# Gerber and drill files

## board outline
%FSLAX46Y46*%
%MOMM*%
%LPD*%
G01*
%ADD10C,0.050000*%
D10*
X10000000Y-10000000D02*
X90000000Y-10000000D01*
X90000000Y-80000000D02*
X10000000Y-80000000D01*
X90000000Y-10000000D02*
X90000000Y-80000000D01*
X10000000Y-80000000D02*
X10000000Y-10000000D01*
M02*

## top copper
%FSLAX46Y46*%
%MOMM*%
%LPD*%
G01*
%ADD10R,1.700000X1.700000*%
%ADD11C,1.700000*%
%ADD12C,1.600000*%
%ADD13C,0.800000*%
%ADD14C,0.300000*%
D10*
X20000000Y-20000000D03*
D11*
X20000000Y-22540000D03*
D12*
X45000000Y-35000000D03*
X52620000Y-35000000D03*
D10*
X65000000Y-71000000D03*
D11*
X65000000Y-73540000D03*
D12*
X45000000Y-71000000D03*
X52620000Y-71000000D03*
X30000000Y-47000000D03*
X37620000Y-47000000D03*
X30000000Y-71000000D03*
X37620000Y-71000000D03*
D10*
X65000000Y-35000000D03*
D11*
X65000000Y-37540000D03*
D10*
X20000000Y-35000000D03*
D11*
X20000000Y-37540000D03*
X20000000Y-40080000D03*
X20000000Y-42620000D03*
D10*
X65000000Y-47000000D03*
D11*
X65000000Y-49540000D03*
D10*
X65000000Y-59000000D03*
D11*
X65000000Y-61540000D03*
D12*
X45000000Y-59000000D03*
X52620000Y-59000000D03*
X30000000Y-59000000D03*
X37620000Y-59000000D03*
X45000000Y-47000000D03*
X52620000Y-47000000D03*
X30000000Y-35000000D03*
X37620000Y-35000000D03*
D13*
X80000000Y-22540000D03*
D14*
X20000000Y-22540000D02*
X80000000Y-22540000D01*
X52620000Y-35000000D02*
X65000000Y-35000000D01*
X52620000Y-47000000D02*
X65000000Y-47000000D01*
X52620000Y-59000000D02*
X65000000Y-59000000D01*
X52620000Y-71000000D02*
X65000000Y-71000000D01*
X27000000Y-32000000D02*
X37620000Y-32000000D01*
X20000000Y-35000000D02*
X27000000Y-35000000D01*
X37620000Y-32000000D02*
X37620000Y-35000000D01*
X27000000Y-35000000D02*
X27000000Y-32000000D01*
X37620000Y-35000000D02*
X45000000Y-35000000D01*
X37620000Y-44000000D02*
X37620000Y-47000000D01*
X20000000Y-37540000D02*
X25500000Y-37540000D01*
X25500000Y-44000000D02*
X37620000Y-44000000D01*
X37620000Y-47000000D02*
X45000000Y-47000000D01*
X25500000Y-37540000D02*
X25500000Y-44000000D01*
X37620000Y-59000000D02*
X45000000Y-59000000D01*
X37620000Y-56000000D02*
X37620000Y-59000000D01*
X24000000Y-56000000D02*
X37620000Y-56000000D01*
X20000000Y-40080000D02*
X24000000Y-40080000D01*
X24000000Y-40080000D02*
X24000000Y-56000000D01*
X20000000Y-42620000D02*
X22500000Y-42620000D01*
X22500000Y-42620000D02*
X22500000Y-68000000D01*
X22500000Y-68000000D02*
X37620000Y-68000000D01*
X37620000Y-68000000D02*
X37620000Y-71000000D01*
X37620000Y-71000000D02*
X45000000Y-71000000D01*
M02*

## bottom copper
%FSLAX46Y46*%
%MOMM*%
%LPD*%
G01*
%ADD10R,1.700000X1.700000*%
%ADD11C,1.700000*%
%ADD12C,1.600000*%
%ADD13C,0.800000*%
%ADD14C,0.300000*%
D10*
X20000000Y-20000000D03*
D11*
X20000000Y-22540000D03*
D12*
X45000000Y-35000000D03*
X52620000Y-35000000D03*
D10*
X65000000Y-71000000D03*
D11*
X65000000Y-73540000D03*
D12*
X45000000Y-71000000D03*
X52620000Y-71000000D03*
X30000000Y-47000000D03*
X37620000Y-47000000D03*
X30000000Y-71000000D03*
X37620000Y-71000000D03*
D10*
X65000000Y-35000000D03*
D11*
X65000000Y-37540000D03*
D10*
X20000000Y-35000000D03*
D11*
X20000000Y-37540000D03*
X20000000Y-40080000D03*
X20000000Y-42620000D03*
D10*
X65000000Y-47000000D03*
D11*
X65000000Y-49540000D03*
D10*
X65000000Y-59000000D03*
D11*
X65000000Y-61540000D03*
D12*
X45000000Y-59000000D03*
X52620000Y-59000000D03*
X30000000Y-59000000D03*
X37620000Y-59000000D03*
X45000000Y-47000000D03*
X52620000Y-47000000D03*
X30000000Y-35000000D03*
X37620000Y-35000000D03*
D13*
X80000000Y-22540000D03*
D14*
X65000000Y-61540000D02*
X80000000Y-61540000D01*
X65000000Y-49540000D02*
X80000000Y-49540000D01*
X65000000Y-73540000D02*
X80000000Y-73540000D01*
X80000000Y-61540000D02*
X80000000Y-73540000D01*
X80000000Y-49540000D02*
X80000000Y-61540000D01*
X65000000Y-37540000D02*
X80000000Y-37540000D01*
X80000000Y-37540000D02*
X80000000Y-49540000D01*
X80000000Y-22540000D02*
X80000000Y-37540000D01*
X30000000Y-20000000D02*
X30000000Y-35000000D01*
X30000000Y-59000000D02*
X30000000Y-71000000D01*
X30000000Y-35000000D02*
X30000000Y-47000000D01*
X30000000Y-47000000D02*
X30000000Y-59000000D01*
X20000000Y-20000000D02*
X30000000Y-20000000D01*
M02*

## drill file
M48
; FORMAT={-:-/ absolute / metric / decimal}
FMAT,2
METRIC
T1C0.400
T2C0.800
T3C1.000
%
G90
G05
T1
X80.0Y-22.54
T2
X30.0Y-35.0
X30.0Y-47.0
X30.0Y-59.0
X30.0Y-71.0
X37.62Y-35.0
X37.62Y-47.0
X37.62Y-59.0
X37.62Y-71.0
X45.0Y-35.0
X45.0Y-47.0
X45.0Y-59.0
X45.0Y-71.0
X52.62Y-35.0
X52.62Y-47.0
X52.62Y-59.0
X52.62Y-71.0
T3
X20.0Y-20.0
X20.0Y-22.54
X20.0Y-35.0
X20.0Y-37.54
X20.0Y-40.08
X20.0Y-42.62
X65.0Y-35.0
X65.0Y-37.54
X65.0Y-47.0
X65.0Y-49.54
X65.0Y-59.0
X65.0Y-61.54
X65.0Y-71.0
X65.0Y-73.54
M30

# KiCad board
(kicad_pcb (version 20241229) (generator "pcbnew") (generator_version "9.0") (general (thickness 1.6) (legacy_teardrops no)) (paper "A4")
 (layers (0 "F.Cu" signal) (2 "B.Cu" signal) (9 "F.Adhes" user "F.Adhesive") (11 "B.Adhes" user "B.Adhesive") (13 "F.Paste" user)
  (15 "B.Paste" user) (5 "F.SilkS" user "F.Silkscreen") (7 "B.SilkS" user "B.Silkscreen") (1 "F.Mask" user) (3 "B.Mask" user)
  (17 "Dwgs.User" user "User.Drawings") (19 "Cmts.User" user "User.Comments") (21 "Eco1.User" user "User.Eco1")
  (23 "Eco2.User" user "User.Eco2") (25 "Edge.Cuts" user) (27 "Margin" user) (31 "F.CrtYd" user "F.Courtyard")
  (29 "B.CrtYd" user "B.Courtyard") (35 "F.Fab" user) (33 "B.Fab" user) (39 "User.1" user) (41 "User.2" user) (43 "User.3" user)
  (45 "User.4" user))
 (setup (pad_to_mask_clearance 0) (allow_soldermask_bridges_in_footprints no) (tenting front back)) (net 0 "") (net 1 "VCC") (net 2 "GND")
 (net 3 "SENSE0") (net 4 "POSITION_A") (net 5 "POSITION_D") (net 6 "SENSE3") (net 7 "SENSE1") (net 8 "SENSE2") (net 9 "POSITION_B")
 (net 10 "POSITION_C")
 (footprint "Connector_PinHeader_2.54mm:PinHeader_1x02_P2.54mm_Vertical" (layer "F.Cu") (at 20 20)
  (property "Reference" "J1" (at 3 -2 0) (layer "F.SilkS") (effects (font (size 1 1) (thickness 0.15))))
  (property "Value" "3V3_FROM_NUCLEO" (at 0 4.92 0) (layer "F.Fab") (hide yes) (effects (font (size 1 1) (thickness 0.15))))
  (pad "1" thru_hole rect (at 0 0) (size 1.7 1.7) (drill 1) (layers "*.Cu" "*.Mask") (remove_unused_layers no) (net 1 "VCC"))
  (pad "2" thru_hole circle (at 0 2.54) (size 1.7 1.7) (drill 1) (layers "*.Cu" "*.Mask") (remove_unused_layers no) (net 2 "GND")))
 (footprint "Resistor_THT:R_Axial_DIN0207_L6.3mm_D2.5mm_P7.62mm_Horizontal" (layer "F.Cu") (at 45 35)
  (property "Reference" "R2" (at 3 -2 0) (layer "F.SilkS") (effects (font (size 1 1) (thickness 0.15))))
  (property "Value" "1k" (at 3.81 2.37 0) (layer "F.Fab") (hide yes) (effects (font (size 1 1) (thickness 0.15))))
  (pad "1" thru_hole circle (at 0 0) (size 1.6 1.6) (drill 0.8) (layers "*.Cu" "*.Mask") (remove_unused_layers no) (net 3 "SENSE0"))
  (pad "2" thru_hole circle (at 7.62 0) (size 1.6 1.6) (drill 0.8) (layers "*.Cu" "*.Mask") (remove_unused_layers no) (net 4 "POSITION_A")))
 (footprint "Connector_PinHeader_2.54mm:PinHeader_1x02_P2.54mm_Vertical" (layer "F.Cu") (at 65 71)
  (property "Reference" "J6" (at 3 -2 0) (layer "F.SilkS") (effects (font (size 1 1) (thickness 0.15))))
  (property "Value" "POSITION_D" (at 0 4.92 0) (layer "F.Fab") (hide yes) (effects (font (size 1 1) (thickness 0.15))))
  (pad "1" thru_hole rect (at 0 0) (size 1.7 1.7) (drill 1) (layers "*.Cu" "*.Mask") (remove_unused_layers no) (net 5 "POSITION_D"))
  (pad "2" thru_hole circle (at 0 2.54) (size 1.7 1.7) (drill 1) (layers "*.Cu" "*.Mask") (remove_unused_layers no) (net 2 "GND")))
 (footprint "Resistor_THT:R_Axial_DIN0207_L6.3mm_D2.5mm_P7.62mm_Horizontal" (layer "F.Cu") (at 45 71)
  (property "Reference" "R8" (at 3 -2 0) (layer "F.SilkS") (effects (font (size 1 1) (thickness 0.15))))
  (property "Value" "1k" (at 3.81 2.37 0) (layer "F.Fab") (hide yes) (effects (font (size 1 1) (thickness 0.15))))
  (pad "1" thru_hole circle (at 0 0) (size 1.6 1.6) (drill 0.8) (layers "*.Cu" "*.Mask") (remove_unused_layers no) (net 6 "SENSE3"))
  (pad "2" thru_hole circle (at 7.62 0) (size 1.6 1.6) (drill 0.8) (layers "*.Cu" "*.Mask") (remove_unused_layers no) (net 5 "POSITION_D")))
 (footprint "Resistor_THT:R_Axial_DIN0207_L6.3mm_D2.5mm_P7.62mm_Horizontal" (layer "F.Cu") (at 30 47)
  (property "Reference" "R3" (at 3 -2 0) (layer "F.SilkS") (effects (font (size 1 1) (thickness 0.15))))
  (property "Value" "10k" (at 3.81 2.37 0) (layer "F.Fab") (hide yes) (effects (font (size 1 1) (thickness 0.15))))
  (pad "1" thru_hole circle (at 0 0) (size 1.6 1.6) (drill 0.8) (layers "*.Cu" "*.Mask") (remove_unused_layers no) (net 1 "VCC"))
  (pad "2" thru_hole circle (at 7.62 0) (size 1.6 1.6) (drill 0.8) (layers "*.Cu" "*.Mask") (remove_unused_layers no) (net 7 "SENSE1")))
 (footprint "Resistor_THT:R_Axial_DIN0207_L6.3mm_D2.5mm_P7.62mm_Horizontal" (layer "F.Cu") (at 30 71)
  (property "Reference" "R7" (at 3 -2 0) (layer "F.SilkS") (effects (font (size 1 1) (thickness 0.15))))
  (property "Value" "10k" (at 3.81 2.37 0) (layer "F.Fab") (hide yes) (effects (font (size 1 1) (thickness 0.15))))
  (pad "1" thru_hole circle (at 0 0) (size 1.6 1.6) (drill 0.8) (layers "*.Cu" "*.Mask") (remove_unused_layers no) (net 1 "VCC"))
  (pad "2" thru_hole circle (at 7.62 0) (size 1.6 1.6) (drill 0.8) (layers "*.Cu" "*.Mask") (remove_unused_layers no) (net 6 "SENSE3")))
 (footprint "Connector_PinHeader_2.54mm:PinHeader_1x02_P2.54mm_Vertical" (layer "F.Cu") (at 65 35)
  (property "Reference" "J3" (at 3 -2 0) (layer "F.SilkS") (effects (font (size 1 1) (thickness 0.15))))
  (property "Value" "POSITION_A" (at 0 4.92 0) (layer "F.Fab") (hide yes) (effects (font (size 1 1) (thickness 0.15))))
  (pad "1" thru_hole rect (at 0 0) (size 1.7 1.7) (drill 1) (layers "*.Cu" "*.Mask") (remove_unused_layers no) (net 4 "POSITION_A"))
  (pad "2" thru_hole circle (at 0 2.54) (size 1.7 1.7) (drill 1) (layers "*.Cu" "*.Mask") (remove_unused_layers no) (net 2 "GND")))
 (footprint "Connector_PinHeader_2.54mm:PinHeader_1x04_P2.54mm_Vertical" (layer "F.Cu") (at 20 35)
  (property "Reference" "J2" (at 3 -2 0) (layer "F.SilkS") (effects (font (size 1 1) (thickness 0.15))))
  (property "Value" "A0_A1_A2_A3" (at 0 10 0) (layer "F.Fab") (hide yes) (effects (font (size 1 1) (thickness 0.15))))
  (pad "1" thru_hole rect (at 0 0) (size 1.7 1.7) (drill 1) (layers "*.Cu" "*.Mask") (remove_unused_layers no) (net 3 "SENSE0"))
  (pad "2" thru_hole circle (at 0 2.54) (size 1.7 1.7) (drill 1) (layers "*.Cu" "*.Mask") (remove_unused_layers no) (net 7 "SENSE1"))
  (pad "3" thru_hole circle (at 0 5.08) (size 1.7 1.7) (drill 1) (layers "*.Cu" "*.Mask") (remove_unused_layers no) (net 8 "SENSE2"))
  (pad "4" thru_hole circle (at 0 7.62) (size 1.7 1.7) (drill 1) (layers "*.Cu" "*.Mask") (remove_unused_layers no) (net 6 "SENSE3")))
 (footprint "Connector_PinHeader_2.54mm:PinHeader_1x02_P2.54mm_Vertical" (layer "F.Cu") (at 65 47)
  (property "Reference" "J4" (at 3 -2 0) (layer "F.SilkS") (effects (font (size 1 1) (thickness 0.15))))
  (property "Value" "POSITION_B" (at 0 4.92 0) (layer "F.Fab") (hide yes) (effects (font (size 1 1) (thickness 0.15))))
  (pad "1" thru_hole rect (at 0 0) (size 1.7 1.7) (drill 1) (layers "*.Cu" "*.Mask") (remove_unused_layers no) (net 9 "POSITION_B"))
  (pad "2" thru_hole circle (at 0 2.54) (size 1.7 1.7) (drill 1) (layers "*.Cu" "*.Mask") (remove_unused_layers no) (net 2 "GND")))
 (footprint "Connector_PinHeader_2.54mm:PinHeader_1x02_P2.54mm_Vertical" (layer "F.Cu") (at 65 59)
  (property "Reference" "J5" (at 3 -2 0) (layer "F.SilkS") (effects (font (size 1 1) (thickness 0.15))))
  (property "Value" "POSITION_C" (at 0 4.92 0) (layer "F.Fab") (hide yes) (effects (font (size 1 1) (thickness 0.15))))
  (pad "1" thru_hole rect (at 0 0) (size 1.7 1.7) (drill 1) (layers "*.Cu" "*.Mask") (remove_unused_layers no) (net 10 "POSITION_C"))
  (pad "2" thru_hole circle (at 0 2.54) (size 1.7 1.7) (drill 1) (layers "*.Cu" "*.Mask") (remove_unused_layers no) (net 2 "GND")))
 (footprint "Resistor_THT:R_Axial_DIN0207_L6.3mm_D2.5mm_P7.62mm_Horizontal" (layer "F.Cu") (at 45 59)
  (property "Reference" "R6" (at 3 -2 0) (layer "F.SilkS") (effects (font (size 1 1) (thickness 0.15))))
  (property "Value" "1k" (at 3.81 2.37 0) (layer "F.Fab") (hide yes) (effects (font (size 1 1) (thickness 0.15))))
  (pad "1" thru_hole circle (at 0 0) (size 1.6 1.6) (drill 0.8) (layers "*.Cu" "*.Mask") (remove_unused_layers no) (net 8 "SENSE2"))
  (pad "2" thru_hole circle (at 7.62 0) (size 1.6 1.6) (drill 0.8) (layers "*.Cu" "*.Mask") (remove_unused_layers no) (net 10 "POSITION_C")))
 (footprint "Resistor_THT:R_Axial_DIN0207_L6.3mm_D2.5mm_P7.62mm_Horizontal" (layer "F.Cu") (at 30 59)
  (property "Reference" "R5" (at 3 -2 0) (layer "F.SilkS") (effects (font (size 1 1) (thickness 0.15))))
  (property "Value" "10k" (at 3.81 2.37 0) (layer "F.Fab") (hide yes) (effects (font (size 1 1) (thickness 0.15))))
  (pad "1" thru_hole circle (at 0 0) (size 1.6 1.6) (drill 0.8) (layers "*.Cu" "*.Mask") (remove_unused_layers no) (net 1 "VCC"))
  (pad "2" thru_hole circle (at 7.62 0) (size 1.6 1.6) (drill 0.8) (layers "*.Cu" "*.Mask") (remove_unused_layers no) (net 8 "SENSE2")))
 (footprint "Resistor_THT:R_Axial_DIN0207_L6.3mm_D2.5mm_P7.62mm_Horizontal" (layer "F.Cu") (at 45 47)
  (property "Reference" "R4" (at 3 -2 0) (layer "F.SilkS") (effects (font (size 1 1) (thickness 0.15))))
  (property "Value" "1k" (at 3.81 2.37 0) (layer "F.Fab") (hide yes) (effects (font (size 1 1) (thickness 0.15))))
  (pad "1" thru_hole circle (at 0 0) (size 1.6 1.6) (drill 0.8) (layers "*.Cu" "*.Mask") (remove_unused_layers no) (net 7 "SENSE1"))
  (pad "2" thru_hole circle (at 7.62 0) (size 1.6 1.6) (drill 0.8) (layers "*.Cu" "*.Mask") (remove_unused_layers no) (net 9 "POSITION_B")))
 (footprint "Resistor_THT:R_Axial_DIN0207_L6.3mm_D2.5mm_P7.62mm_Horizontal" (layer "F.Cu") (at 30 35)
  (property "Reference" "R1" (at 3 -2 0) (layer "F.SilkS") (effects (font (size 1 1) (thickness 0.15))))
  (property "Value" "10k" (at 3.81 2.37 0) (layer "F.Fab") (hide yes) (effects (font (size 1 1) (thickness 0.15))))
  (pad "1" thru_hole circle (at 0 0) (size 1.6 1.6) (drill 0.8) (layers "*.Cu" "*.Mask") (remove_unused_layers no) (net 1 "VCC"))
  (pad "2" thru_hole circle (at 7.62 0) (size 1.6 1.6) (drill 0.8) (layers "*.Cu" "*.Mask") (remove_unused_layers no) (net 3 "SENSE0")))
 (gr_line (start 10 10) (end 90 10) (stroke (width 0.05) (type default)) (layer "Edge.Cuts"))
 (gr_line (start 90 80) (end 10 80) (stroke (width 0.05) (type default)) (layer "Edge.Cuts"))
 (gr_line (start 90 10) (end 90 80) (stroke (width 0.05) (type default)) (layer "Edge.Cuts"))
 (gr_line (start 10 80) (end 10 10) (stroke (width 0.05) (type default)) (layer "Edge.Cuts"))
 (segment (start 20 22.54) (end 80 22.54) (width 0.3) (layer "F.Cu") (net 2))
 (via (at 80 22.54) (size 0.8) (drill 0.4) (layers "F.Cu" "B.Cu") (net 2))
 (segment (start 65 61.54) (end 80 61.54) (width 0.3) (layer "B.Cu") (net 2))
 (segment (start 65 49.54) (end 80 49.54) (width 0.3) (layer "B.Cu") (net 2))
 (segment (start 65 73.54) (end 80 73.54) (width 0.3) (layer "B.Cu") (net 2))
 (segment (start 80 61.54) (end 80 73.54) (width 0.3) (layer "B.Cu") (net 2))
 (segment (start 80 49.54) (end 80 61.54) (width 0.3) (layer "B.Cu") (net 2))
 (segment (start 65 37.54) (end 80 37.54) (width 0.3) (layer "B.Cu") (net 2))
 (segment (start 80 37.54) (end 80 49.54) (width 0.3) (layer "B.Cu") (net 2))
 (segment (start 80 22.54) (end 80 37.54) (width 0.3) (layer "B.Cu") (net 2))
 (segment (start 52.62 35) (end 65 35) (width 0.3) (layer "F.Cu") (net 4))
 (segment (start 52.62 47) (end 65 47) (width 0.3) (layer "F.Cu") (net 9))
 (segment (start 52.62 59) (end 65 59) (width 0.3) (layer "F.Cu") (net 10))
 (segment (start 52.62 71) (end 65 71) (width 0.3) (layer "F.Cu") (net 5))
 (segment (start 27 32) (end 37.62 32) (width 0.3) (layer "F.Cu") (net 3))
 (segment (start 20 35) (end 27 35) (width 0.3) (layer "F.Cu") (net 3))
 (segment (start 37.62 32) (end 37.62 35) (width 0.3) (layer "F.Cu") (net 3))
 (segment (start 27 35) (end 27 32) (width 0.3) (layer "F.Cu") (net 3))
 (segment (start 37.62 35) (end 45 35) (width 0.3) (layer "F.Cu") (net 3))
 (segment (start 37.62 44) (end 37.62 47) (width 0.3) (layer "F.Cu") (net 7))
 (segment (start 20 37.54) (end 25.5 37.54) (width 0.3) (layer "F.Cu") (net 7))
 (segment (start 25.5 44) (end 37.62 44) (width 0.3) (layer "F.Cu") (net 7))
 (segment (start 37.62 47) (end 45 47) (width 0.3) (layer "F.Cu") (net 7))
 (segment (start 25.5 37.54) (end 25.5 44) (width 0.3) (layer "F.Cu") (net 7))
 (segment (start 37.62 59) (end 45 59) (width 0.3) (layer "F.Cu") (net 8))
 (segment (start 37.62 56) (end 37.62 59) (width 0.3) (layer "F.Cu") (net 8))
 (segment (start 24 56) (end 37.62 56) (width 0.3) (layer "F.Cu") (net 8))
 (segment (start 20 40.08) (end 24 40.08) (width 0.3) (layer "F.Cu") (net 8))
 (segment (start 24 40.08) (end 24 56) (width 0.3) (layer "F.Cu") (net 8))
 (segment (start 20 42.62) (end 22.5 42.62) (width 0.3) (layer "F.Cu") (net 6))
 (segment (start 22.5 42.62) (end 22.5 68) (width 0.3) (layer "F.Cu") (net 6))
 (segment (start 22.5 68) (end 37.62 68) (width 0.3) (layer "F.Cu") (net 6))
 (segment (start 37.62 68) (end 37.62 71) (width 0.3) (layer "F.Cu") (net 6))
 (segment (start 37.62 71) (end 45 71) (width 0.3) (layer "F.Cu") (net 6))
 (segment (start 30 20) (end 30 35) (width 0.3) (layer "B.Cu") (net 1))
 (segment (start 30 59) (end 30 71) (width 0.3) (layer "B.Cu") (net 1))
 (segment (start 30 35) (end 30 47) (width 0.3) (layer "B.Cu") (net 1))
 (segment (start 30 47) (end 30 59) (width 0.3) (layer "B.Cu") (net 1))
 (segment (start 20 20) (end 30 20) (width 0.3) (layer "B.Cu") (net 1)))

